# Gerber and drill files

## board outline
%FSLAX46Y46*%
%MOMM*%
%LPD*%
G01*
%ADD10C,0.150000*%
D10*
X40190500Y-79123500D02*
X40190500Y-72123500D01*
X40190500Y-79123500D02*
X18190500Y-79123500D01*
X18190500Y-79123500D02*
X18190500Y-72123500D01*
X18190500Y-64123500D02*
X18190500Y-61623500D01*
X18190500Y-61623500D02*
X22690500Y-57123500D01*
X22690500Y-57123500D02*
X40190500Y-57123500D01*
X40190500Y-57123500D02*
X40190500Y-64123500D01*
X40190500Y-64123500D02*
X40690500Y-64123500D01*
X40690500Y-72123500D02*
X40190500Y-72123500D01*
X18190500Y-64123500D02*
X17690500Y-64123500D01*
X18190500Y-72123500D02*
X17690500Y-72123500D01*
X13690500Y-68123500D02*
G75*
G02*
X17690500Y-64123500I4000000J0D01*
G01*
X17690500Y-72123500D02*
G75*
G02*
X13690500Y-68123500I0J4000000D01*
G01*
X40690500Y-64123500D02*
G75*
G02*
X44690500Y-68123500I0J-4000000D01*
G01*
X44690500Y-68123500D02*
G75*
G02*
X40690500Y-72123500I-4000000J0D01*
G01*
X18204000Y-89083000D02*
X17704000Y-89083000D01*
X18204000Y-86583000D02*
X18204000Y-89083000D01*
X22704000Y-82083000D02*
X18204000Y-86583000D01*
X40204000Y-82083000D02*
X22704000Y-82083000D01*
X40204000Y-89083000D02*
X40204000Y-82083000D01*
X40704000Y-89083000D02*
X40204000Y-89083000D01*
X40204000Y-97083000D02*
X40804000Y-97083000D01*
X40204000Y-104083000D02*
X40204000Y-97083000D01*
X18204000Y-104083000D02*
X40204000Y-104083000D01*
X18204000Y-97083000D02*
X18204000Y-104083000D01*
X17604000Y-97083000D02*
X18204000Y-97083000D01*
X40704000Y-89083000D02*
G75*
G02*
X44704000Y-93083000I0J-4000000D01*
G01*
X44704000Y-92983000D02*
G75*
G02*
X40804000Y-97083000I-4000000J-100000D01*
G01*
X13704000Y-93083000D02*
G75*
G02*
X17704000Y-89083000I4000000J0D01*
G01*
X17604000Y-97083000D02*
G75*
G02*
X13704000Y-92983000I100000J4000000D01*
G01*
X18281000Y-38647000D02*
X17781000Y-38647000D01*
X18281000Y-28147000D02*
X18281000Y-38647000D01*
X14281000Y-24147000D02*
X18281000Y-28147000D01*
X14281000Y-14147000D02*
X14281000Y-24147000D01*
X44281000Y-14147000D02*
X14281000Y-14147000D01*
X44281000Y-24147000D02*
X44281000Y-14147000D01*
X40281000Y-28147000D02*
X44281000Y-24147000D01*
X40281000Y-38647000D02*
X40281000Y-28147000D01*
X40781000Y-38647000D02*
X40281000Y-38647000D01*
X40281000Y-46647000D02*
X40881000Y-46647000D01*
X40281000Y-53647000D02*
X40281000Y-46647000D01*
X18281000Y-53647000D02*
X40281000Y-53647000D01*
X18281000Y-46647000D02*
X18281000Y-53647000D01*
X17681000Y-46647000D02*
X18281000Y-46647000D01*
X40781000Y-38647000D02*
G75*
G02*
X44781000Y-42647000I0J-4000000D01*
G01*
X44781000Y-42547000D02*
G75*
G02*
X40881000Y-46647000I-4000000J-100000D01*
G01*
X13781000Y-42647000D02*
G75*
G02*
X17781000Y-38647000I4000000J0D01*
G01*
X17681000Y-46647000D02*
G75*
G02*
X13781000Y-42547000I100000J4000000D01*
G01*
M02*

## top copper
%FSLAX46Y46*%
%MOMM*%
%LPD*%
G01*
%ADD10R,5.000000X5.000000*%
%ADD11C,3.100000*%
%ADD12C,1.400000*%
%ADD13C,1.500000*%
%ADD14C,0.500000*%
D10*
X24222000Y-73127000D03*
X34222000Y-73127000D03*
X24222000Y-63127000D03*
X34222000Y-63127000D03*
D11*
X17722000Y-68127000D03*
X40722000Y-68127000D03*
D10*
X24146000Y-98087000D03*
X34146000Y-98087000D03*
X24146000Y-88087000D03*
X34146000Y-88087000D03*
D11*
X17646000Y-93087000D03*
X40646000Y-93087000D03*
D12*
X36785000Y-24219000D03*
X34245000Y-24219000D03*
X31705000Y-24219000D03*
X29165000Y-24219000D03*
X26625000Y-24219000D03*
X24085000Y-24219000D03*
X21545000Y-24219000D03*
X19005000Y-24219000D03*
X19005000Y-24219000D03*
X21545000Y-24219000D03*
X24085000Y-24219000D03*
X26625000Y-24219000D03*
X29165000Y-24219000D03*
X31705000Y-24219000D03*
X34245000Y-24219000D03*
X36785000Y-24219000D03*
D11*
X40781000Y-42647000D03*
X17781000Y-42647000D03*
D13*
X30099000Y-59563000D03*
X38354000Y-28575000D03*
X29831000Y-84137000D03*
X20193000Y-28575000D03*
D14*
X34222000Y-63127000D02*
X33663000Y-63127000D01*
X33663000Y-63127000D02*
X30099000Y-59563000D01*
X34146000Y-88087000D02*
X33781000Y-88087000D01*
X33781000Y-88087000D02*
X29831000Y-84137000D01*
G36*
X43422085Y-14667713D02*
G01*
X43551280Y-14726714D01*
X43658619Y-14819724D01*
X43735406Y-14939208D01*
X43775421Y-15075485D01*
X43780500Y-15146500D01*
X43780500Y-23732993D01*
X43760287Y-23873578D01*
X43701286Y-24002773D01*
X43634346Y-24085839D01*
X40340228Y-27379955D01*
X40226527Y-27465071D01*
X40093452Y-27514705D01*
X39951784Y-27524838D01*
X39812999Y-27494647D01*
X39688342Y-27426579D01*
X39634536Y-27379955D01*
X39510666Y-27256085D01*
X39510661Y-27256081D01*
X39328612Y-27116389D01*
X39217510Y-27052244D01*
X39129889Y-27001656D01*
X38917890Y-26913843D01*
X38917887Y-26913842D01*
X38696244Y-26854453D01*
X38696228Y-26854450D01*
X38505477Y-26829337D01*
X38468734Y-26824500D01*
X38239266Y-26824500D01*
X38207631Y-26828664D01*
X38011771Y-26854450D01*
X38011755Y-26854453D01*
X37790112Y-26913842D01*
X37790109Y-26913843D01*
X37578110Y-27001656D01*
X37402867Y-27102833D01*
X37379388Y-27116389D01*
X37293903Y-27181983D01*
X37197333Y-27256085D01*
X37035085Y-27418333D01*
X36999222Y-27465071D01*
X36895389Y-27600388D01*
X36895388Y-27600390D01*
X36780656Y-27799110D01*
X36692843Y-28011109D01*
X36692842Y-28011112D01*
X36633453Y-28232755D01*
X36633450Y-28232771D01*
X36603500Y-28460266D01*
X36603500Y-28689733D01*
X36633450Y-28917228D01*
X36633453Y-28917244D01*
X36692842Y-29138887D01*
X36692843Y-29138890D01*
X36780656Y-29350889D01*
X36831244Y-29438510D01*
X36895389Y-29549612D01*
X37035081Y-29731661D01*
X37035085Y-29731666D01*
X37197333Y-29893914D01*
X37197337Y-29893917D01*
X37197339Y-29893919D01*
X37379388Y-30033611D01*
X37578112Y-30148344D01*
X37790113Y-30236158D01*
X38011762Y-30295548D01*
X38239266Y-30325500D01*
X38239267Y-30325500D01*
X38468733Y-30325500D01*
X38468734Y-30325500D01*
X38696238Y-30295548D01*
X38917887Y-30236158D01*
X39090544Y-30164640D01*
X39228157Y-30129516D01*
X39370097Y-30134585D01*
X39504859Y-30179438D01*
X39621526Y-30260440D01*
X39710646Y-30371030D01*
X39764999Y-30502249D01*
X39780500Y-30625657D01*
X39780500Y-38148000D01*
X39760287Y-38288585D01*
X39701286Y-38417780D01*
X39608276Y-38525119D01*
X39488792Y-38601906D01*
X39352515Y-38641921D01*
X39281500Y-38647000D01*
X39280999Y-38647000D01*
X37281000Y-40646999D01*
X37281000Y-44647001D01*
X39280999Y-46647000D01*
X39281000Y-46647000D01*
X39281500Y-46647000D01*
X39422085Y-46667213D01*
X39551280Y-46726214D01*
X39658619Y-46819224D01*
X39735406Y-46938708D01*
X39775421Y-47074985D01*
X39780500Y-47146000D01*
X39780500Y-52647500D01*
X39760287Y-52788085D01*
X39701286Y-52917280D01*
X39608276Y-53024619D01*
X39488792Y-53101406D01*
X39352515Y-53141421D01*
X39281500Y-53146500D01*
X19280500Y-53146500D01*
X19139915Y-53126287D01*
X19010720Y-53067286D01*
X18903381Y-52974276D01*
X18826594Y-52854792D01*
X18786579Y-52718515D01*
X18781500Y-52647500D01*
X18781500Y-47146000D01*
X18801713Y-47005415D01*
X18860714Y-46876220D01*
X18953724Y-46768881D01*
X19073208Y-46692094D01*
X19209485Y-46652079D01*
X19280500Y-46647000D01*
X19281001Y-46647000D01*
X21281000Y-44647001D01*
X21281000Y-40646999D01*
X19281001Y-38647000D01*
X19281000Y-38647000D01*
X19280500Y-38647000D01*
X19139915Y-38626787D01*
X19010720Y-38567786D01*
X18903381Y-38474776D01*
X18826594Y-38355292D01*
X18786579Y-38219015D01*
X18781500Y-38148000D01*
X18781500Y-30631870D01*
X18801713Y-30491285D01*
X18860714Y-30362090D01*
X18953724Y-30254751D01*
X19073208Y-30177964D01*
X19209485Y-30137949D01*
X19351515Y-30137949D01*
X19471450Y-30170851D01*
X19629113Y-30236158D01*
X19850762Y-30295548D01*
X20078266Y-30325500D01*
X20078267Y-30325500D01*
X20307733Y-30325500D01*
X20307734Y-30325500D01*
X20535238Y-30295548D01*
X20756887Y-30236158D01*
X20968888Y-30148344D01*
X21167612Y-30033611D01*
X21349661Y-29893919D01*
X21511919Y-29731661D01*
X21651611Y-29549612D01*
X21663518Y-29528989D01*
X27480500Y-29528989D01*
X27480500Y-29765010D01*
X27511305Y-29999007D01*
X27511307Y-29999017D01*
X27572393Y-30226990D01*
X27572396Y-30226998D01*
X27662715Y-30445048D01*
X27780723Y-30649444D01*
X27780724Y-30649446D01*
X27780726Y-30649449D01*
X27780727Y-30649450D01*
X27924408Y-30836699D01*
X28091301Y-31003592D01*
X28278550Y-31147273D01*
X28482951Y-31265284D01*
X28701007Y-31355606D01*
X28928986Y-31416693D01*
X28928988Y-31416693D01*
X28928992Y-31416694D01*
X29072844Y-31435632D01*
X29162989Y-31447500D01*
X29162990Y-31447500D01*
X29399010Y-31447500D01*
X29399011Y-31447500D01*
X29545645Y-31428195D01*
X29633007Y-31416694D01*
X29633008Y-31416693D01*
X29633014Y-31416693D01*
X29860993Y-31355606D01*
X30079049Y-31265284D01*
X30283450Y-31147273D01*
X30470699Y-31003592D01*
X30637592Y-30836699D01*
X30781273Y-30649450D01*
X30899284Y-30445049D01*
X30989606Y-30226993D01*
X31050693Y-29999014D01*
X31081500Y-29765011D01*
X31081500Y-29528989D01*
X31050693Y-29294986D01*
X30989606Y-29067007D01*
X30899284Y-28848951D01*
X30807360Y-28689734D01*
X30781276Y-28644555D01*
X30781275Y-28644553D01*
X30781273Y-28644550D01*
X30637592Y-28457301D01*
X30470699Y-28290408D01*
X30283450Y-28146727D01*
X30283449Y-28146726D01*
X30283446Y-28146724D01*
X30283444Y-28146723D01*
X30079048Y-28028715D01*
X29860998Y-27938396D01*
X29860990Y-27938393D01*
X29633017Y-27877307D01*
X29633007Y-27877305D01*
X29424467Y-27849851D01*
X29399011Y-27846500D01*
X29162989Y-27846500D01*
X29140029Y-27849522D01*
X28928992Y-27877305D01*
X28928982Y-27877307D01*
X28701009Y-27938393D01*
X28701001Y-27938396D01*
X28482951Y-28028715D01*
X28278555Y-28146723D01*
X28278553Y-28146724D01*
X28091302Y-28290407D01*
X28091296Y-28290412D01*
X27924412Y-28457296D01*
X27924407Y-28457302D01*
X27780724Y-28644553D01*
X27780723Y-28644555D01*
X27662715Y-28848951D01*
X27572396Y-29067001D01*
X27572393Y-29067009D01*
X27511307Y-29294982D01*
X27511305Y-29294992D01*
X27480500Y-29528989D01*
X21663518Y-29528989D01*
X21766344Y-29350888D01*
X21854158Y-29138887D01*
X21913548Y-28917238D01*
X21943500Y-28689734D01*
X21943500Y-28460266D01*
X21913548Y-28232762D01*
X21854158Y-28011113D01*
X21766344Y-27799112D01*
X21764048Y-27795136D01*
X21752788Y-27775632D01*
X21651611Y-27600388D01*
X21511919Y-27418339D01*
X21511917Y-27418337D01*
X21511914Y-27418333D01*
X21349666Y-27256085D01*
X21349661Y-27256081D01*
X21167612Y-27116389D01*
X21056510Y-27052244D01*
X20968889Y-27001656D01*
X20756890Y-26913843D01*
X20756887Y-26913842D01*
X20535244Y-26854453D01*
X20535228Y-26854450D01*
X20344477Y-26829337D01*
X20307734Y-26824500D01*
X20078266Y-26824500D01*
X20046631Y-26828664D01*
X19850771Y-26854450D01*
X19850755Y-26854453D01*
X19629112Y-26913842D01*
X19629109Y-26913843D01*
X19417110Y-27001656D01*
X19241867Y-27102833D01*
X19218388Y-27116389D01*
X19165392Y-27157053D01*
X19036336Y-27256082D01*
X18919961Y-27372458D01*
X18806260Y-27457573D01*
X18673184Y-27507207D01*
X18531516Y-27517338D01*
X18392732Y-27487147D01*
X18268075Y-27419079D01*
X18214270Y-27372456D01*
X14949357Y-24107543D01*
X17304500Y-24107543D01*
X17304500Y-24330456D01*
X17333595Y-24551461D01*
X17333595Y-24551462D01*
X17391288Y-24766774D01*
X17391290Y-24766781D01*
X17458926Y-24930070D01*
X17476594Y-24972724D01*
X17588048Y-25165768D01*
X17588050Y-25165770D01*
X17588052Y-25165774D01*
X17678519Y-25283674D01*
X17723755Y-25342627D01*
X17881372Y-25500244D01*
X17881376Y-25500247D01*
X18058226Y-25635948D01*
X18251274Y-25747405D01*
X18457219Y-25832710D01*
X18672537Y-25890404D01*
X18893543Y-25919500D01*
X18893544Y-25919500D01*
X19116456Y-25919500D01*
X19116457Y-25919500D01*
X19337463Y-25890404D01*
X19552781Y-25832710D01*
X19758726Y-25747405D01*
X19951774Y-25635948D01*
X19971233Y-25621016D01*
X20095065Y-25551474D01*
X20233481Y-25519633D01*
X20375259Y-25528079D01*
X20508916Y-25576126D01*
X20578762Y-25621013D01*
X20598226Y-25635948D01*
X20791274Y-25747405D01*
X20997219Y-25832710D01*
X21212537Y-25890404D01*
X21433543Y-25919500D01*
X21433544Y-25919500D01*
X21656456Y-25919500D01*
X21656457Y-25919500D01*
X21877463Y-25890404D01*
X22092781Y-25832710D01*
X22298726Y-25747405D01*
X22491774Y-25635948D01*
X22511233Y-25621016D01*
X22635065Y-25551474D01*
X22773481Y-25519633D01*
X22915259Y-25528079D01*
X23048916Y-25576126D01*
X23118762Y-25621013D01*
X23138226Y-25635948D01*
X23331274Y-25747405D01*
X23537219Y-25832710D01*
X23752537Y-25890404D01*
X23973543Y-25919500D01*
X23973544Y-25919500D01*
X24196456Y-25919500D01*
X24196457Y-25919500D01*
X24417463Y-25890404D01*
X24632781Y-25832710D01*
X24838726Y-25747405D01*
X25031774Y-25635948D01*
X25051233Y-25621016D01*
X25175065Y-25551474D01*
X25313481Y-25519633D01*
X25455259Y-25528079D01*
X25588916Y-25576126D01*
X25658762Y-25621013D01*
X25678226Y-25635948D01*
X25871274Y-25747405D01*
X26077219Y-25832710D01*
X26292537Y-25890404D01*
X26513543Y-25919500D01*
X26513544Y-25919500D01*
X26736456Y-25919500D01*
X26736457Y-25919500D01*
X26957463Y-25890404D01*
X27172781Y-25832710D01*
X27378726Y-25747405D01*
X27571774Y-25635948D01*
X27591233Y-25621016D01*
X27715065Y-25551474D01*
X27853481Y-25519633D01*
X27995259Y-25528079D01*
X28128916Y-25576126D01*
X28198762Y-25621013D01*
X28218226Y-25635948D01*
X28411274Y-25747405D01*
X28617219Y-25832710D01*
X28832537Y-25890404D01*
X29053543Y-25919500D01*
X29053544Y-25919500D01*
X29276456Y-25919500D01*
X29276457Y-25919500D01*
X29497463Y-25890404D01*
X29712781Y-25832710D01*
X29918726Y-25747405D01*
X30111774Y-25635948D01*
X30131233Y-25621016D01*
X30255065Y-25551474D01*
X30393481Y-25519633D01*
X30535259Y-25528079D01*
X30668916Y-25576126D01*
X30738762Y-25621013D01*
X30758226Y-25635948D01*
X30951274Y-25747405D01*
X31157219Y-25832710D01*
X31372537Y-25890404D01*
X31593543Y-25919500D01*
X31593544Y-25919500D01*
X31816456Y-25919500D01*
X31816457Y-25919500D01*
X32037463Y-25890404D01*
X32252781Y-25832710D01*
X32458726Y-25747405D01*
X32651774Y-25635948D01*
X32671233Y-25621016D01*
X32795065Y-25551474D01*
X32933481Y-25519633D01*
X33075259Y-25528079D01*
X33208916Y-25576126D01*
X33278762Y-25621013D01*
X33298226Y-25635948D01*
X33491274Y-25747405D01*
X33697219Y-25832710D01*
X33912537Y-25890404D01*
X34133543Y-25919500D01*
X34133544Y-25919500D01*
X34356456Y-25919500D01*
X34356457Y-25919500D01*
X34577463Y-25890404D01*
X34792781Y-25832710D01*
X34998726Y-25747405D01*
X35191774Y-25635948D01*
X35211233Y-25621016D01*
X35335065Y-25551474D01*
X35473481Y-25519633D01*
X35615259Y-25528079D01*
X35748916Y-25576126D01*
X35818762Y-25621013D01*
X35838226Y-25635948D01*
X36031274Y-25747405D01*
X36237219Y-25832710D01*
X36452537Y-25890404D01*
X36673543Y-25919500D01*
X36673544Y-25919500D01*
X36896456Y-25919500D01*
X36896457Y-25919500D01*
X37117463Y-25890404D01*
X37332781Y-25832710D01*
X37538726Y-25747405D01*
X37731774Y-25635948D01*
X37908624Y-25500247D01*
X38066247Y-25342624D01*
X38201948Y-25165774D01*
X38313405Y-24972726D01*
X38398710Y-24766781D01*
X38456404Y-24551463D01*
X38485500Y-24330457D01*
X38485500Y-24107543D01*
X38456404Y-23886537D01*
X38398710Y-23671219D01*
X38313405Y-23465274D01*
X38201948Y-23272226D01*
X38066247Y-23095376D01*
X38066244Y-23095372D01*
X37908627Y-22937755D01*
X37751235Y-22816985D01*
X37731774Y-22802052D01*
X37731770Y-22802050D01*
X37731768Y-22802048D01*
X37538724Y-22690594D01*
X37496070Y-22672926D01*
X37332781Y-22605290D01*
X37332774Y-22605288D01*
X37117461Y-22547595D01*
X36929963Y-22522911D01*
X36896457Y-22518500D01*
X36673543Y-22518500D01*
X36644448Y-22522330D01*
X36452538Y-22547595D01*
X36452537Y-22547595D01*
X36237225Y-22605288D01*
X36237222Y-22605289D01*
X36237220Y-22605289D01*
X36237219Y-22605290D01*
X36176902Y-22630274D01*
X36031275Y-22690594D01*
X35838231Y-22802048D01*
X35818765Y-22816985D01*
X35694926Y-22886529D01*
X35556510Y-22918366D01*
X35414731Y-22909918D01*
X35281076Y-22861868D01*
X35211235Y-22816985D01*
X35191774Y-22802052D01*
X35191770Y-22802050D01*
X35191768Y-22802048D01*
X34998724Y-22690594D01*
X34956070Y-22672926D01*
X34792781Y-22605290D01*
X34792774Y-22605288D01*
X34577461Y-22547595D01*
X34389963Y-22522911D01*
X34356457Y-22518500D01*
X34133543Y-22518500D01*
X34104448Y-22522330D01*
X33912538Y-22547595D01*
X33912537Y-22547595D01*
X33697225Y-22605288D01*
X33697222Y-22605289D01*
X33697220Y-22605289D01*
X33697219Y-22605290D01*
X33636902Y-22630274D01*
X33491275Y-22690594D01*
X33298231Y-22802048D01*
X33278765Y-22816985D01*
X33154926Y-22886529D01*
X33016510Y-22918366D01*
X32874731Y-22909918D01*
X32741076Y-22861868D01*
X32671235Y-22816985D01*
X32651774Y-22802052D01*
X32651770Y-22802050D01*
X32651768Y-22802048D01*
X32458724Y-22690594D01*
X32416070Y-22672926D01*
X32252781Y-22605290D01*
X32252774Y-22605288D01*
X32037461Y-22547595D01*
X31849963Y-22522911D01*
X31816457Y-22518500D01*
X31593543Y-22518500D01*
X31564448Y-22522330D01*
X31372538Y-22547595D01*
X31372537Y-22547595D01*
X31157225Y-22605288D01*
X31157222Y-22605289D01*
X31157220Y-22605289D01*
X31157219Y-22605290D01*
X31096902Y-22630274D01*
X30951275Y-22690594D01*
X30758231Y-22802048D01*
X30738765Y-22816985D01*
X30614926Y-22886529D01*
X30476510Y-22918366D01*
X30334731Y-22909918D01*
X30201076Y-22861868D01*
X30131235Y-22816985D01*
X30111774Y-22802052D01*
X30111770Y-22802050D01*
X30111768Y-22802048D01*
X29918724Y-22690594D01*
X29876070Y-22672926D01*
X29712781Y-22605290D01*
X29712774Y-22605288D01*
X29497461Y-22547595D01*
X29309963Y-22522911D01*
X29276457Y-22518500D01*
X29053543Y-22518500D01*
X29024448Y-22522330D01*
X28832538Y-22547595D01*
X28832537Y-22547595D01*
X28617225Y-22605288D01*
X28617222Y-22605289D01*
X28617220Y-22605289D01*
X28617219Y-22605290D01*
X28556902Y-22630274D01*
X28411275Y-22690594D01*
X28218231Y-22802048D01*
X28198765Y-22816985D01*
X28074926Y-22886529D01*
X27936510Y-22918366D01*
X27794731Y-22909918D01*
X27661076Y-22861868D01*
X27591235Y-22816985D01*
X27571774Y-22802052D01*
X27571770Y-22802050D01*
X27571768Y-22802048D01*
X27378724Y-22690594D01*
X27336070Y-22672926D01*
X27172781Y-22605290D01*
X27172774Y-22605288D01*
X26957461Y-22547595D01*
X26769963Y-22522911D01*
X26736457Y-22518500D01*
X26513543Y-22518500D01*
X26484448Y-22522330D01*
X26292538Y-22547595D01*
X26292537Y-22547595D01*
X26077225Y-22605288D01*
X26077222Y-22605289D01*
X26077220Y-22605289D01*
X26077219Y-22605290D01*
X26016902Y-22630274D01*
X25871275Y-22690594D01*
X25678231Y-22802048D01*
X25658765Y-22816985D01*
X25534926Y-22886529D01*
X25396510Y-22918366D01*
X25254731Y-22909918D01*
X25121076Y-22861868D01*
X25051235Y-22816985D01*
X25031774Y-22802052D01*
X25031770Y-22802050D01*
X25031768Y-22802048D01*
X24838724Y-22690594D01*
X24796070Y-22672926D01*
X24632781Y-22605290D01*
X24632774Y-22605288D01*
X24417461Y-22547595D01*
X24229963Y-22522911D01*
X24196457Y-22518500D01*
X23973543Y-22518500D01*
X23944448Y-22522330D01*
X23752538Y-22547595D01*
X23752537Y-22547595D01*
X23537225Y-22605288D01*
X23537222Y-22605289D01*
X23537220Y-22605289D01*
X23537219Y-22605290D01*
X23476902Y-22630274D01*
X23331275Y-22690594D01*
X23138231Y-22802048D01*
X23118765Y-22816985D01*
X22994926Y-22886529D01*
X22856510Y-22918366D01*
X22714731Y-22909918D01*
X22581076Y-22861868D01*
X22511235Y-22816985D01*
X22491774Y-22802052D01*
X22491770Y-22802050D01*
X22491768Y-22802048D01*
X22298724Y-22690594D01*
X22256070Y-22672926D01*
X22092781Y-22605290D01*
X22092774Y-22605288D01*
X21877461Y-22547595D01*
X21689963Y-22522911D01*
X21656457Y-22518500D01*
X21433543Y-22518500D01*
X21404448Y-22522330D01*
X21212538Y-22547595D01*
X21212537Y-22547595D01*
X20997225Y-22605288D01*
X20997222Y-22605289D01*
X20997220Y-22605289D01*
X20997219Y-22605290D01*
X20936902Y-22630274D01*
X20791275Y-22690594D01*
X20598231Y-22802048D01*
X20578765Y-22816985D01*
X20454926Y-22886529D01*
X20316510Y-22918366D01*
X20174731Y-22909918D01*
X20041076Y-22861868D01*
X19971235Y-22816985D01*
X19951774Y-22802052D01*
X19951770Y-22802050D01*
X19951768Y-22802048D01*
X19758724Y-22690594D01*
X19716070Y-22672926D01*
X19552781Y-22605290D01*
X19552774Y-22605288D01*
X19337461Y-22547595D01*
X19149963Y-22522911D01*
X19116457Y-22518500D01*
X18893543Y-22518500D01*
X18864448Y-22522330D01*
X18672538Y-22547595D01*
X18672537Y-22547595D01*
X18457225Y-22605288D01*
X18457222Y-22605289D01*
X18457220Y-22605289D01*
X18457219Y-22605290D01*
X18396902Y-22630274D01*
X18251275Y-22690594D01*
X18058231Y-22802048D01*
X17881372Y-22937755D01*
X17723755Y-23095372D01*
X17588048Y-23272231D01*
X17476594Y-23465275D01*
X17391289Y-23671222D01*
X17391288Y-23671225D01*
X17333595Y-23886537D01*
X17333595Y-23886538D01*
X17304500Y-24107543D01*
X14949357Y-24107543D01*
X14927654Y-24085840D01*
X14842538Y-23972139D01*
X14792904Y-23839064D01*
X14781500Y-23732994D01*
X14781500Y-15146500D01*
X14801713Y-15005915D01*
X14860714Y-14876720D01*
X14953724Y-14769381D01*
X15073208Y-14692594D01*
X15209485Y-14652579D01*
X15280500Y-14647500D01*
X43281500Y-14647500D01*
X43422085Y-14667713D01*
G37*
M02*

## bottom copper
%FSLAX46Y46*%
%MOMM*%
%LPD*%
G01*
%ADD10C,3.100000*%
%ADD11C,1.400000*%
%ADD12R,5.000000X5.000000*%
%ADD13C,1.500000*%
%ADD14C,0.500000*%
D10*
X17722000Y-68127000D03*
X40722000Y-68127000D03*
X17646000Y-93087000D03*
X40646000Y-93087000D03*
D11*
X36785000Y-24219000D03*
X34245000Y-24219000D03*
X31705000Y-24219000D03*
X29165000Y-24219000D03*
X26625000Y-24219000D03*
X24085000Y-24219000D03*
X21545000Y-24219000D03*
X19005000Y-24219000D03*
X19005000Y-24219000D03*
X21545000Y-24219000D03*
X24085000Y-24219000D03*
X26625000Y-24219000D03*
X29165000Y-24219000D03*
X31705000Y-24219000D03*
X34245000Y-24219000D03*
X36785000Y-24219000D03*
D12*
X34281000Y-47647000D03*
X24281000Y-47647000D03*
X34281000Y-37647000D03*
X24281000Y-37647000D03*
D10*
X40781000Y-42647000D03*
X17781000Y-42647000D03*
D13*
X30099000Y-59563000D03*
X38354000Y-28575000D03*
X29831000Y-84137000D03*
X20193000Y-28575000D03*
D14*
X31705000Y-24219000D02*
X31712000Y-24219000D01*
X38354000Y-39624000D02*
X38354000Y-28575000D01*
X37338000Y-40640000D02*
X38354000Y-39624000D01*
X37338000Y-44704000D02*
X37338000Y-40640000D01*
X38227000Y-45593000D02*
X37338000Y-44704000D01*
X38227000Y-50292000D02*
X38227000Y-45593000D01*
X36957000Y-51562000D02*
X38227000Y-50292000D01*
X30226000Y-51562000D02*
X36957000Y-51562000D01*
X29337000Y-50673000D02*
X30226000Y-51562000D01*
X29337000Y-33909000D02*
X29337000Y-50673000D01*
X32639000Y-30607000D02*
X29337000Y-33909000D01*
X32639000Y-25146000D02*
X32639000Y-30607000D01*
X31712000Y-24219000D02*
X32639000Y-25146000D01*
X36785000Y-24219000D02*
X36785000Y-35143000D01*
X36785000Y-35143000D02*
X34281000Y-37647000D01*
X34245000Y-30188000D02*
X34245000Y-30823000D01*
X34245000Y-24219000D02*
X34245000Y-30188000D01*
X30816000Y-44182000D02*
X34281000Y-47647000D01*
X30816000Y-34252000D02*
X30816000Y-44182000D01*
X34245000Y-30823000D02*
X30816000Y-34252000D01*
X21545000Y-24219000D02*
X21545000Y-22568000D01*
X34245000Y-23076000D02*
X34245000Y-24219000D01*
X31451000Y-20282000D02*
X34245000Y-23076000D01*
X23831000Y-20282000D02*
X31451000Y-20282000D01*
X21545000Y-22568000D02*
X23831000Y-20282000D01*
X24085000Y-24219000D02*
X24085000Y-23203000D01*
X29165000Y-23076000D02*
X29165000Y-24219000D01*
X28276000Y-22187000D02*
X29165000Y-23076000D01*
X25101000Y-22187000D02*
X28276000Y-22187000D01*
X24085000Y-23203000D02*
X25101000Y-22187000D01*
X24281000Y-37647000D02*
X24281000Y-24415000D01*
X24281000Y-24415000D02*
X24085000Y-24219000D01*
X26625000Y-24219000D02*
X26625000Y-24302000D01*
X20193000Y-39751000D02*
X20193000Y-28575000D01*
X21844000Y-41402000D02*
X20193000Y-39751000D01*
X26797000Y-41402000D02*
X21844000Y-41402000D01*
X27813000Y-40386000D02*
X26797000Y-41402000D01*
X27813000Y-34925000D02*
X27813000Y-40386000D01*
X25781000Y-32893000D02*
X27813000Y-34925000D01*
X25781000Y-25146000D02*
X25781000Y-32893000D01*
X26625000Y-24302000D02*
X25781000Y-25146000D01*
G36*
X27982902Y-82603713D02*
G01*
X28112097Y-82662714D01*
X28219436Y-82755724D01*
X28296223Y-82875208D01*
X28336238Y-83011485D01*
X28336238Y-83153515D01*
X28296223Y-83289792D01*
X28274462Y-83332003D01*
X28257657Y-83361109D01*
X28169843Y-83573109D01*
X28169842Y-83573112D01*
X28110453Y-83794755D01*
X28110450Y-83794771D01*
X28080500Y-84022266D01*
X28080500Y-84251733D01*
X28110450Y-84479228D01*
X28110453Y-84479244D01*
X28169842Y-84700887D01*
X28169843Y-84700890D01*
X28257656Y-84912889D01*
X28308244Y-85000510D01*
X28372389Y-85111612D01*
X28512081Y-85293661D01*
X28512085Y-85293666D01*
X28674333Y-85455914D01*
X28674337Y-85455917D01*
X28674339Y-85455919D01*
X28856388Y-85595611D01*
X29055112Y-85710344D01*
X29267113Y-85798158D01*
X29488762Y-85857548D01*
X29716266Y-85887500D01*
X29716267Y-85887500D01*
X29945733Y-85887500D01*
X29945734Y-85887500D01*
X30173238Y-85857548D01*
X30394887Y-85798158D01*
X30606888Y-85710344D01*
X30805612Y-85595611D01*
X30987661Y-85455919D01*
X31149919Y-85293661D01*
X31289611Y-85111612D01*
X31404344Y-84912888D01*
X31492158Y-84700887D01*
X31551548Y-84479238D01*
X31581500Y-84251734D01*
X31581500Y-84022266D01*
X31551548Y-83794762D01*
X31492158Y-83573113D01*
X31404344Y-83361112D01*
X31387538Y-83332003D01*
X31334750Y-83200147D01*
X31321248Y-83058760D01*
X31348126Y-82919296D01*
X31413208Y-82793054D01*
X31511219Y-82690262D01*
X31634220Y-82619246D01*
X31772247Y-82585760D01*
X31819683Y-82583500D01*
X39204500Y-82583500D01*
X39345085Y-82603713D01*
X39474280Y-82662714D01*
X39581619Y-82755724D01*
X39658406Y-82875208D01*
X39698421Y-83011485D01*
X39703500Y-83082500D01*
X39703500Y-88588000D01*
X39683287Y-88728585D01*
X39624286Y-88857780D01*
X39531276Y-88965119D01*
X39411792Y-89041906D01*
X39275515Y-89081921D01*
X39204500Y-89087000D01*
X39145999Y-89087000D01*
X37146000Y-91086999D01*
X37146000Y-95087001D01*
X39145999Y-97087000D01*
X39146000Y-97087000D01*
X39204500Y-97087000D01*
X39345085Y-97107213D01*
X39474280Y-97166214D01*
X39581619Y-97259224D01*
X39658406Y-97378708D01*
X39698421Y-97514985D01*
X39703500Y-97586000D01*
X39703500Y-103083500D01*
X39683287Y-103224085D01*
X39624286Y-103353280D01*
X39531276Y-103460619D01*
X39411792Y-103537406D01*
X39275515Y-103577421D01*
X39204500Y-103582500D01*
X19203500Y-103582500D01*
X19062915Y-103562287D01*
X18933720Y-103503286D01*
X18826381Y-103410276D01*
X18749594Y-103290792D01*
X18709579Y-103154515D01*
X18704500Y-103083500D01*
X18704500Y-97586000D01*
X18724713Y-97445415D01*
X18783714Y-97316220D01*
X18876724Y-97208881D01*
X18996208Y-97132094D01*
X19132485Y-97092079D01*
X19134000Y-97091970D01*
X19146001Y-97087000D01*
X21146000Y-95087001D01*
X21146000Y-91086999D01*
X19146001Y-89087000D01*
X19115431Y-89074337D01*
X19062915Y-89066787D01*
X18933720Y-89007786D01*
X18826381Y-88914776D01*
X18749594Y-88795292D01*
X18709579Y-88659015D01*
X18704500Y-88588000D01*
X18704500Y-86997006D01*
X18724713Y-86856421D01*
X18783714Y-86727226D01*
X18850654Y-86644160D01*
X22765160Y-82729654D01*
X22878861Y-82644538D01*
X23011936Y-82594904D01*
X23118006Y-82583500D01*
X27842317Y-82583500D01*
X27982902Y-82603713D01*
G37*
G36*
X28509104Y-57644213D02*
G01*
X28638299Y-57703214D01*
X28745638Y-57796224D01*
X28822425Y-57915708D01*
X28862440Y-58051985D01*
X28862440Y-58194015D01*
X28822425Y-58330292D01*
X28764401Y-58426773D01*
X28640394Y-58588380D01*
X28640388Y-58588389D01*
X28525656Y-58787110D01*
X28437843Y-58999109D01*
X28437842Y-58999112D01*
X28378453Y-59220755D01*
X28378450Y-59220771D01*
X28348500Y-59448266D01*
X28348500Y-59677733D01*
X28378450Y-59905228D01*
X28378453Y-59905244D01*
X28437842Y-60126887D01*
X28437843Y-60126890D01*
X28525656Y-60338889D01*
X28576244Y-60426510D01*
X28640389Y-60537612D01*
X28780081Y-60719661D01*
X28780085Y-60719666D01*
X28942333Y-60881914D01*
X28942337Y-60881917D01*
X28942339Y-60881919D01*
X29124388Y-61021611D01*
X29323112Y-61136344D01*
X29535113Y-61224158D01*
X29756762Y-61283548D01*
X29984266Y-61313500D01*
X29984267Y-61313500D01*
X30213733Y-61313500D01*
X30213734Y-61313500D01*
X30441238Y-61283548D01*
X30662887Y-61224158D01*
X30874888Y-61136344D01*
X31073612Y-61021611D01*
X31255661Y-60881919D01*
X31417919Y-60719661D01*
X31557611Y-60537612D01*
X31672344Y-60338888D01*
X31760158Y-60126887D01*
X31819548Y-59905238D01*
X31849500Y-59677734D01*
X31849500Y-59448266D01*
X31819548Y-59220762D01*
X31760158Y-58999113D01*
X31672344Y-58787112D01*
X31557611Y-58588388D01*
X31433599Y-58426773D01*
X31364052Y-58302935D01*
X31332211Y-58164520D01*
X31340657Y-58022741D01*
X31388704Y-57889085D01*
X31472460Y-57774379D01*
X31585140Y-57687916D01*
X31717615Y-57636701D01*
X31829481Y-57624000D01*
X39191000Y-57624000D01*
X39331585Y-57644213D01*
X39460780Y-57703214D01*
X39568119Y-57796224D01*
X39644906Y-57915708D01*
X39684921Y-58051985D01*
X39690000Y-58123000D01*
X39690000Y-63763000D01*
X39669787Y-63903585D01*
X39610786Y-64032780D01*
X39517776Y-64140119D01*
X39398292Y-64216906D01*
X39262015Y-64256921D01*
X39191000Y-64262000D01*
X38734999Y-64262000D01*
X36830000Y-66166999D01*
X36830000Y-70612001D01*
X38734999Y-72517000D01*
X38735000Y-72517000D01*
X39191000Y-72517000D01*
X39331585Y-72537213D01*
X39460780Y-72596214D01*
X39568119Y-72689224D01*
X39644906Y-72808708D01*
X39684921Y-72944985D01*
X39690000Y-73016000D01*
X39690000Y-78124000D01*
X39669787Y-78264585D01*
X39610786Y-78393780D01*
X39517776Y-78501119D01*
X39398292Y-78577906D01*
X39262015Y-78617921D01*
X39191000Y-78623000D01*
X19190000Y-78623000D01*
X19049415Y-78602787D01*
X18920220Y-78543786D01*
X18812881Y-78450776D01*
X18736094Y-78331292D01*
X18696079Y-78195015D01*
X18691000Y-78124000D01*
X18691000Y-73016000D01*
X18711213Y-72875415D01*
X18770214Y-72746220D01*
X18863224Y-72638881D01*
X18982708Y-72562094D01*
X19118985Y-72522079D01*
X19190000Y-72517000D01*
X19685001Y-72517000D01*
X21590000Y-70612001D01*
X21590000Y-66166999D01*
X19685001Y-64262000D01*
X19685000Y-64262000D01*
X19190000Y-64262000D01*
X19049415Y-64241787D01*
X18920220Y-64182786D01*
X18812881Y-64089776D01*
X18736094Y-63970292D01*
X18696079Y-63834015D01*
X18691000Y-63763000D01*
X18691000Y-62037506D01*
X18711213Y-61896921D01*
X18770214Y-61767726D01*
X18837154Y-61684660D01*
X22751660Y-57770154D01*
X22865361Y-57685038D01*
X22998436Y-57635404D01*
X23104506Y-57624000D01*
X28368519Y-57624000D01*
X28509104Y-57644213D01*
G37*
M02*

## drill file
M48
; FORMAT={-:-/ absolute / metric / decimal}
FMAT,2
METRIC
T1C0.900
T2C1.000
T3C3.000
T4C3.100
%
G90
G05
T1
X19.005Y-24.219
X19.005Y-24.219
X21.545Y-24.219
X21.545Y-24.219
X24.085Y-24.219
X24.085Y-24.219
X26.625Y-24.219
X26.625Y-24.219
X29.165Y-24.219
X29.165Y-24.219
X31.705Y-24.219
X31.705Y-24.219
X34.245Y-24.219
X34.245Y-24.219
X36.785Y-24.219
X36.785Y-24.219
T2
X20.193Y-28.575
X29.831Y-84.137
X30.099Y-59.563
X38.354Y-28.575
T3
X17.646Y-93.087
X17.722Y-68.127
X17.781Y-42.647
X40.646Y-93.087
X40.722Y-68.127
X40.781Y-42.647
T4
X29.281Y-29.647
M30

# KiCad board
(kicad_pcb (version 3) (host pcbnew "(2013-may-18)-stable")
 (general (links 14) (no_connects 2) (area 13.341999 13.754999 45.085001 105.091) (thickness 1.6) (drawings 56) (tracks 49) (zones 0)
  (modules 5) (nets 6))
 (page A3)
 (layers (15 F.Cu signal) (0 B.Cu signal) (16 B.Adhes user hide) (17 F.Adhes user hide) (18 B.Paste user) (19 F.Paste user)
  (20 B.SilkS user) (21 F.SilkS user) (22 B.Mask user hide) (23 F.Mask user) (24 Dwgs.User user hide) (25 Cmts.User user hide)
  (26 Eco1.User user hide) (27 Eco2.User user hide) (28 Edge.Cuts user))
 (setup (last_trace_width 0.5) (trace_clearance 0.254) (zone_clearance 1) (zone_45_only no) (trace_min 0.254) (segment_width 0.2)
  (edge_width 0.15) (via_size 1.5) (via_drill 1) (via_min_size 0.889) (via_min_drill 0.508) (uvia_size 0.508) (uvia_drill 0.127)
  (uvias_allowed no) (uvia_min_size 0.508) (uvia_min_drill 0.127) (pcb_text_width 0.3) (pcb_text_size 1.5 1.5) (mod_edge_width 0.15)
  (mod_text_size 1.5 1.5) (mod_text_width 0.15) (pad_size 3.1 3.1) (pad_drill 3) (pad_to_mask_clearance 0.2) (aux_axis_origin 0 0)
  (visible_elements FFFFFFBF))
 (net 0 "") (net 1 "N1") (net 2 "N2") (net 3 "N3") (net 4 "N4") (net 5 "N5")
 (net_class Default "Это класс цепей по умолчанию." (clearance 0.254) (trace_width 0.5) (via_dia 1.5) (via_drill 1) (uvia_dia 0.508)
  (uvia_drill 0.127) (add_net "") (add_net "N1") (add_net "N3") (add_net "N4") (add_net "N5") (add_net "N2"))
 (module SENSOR (layer F.Cu) (at 17.722 79.627)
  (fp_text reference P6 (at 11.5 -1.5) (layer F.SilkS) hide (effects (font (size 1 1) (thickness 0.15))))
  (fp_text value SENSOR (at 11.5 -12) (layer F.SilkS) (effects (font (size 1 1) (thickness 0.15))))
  (pad 2 smd rect (at 6.5 -6.5) (size 5 5) (layers F.Cu F.Mask) (solder_mask_margin 0.1))
  (pad 3 smd rect (at 16.5 -6.5) (size 5 5) (layers F.Cu F.Mask))
  (pad 1 smd rect (at 6.5 -16.5) (size 5 5) (layers F.Cu F.Mask))
  (pad 4 smd rect (at 16.5 -16.5) (size 5 5) (layers F.Cu F.Mask) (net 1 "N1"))
  (pad "" np_thru_hole circle (at 0 -11.5) (size 3.1 3.1) (drill 3) (layers *.Cu *.Mask F.SilkS))
  (pad "" np_thru_hole circle (at 23 -11.5) (size 3.1 3.1) (drill 3) (layers *.Cu *.Mask F.SilkS)))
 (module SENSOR (layer F.Cu) (at 17.646 104.587)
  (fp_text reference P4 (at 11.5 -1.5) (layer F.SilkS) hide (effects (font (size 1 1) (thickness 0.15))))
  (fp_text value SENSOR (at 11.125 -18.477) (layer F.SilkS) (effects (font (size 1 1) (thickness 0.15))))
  (pad 2 smd rect (at 6.5 -6.5) (size 5 5) (layers F.Cu F.Mask) (solder_mask_margin 0.1))
  (pad 3 smd rect (at 16.5 -6.5) (size 5 5) (layers F.Cu F.Mask))
  (pad 1 smd rect (at 6.5 -16.5) (size 5 5) (layers F.Cu F.Mask))
  (pad 4 smd rect (at 16.5 -16.5) (size 5 5) (layers F.Cu F.Mask) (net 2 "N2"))
  (pad "" np_thru_hole circle (at 0 -11.5) (size 3.1 3.1) (drill 3) (layers *.Cu *.Mask F.SilkS))
  (pad "" np_thru_hole circle (at 23 -11.5) (size 3.1 3.1) (drill 3) (layers *.Cu *.Mask F.SilkS)))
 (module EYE (layer F.Cu) (at 27.895 24.219 270)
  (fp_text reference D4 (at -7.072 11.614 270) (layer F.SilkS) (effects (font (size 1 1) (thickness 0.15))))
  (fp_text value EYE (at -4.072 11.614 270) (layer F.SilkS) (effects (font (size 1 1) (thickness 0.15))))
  (pad 1 thru_hole circle (at 0 -8.89 270) (size 1.4 1.4) (drill 0.9) (layers *.Cu *.Mask F.SilkS) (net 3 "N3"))
  (pad 2 thru_hole circle (at 0 -6.35 270) (size 1.4 1.4) (drill 0.9) (layers *.Cu *.Mask F.SilkS) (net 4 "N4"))
  (pad 3 thru_hole circle (at 0 -3.81 270) (size 1.4 1.4) (drill 0.9) (layers *.Cu *.Mask F.SilkS) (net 1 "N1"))
  (pad 4 thru_hole circle (at 0 -1.27 270) (size 1.4 1.4) (drill 0.9) (layers *.Cu *.Mask F.SilkS) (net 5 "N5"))
  (pad 5 thru_hole circle (at 0 1.27 270) (size 1.4 1.4) (drill 0.9) (layers *.Cu *.Mask F.SilkS) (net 2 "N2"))
  (pad 6 thru_hole circle (at 0 3.81 270) (size 1.4 1.4) (drill 0.9) (layers *.Cu *.Mask F.SilkS) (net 5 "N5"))
  (pad 7 thru_hole circle (at 0 6.35 270) (size 1.4 1.4) (drill 0.9) (layers *.Cu *.Mask F.SilkS) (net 4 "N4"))
  (pad 8 thru_hole circle (at 0 8.89 270) (size 1.4 1.4) (drill 0.9) (layers *.Cu *.Mask F.SilkS))
  (pad 8 thru_hole circle (at 0 8.89 270) (size 1.4 1.4) (drill 0.9) (layers *.Cu *.Mask F.SilkS))
  (pad 7 thru_hole circle (at 0 6.35 270) (size 1.4 1.4) (drill 0.9) (layers *.Cu *.Mask F.SilkS) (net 4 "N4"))
  (pad 6 thru_hole circle (at 0 3.81 270) (size 1.4 1.4) (drill 0.9) (layers *.Cu *.Mask F.SilkS) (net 5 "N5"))
  (pad 5 thru_hole circle (at 0 1.27 270) (size 1.4 1.4) (drill 0.9) (layers *.Cu *.Mask F.SilkS) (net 2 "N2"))
  (pad 4 thru_hole circle (at 0 -1.27 270) (size 1.4 1.4) (drill 0.9) (layers *.Cu *.Mask F.SilkS) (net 5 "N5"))
  (pad 3 thru_hole circle (at 0 -3.81 270) (size 1.4 1.4) (drill 0.9) (layers *.Cu *.Mask F.SilkS) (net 1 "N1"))
  (pad 2 thru_hole circle (at 0 -6.35 270) (size 1.4 1.4) (drill 0.9) (layers *.Cu *.Mask F.SilkS) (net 4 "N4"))
  (pad 1 thru_hole circle (at 0 -8.89 270) (size 1.4 1.4) (drill 0.9) (layers *.Cu *.Mask F.SilkS) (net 3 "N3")))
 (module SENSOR (layer B.Cu) (at 40.781 54.147 180)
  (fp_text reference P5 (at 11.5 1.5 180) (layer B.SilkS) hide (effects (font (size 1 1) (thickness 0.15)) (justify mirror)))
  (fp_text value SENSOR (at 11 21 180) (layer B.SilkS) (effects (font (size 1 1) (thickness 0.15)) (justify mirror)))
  (pad 2 smd rect (at 6.5 6.5 180) (size 5 5) (layers B.Cu B.Mask) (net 4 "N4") (solder_mask_margin 0.1))
  (pad 3 smd rect (at 16.5 6.5 180) (size 5 5) (layers B.Cu B.Mask))
  (pad 1 smd rect (at 6.5 16.5 180) (size 5 5) (layers B.Cu B.Mask) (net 3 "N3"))
  (pad 4 smd rect (at 16.5 16.5 180) (size 5 5) (layers B.Cu B.Mask) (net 5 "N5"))
  (pad "" np_thru_hole circle (at 0 11.5 180) (size 3.1 3.1) (drill 3) (layers *.Cu *.Mask B.SilkS))
  (pad "" np_thru_hole circle (at 23 11.5 180) (size 3.1 3.1) (drill 3) (layers *.Cu *.Mask B.SilkS)))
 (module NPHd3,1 (layer F.Cu) (at 29.281 29.647 90)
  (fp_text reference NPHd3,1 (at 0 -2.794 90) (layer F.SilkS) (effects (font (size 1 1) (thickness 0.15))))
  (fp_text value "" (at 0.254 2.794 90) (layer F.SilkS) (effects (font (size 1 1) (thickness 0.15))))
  (pad "" np_thru_hole circle (at 0 0 90) (size 3.1 3.1) (drill 3.1) (layers *.Cu *.Mask F.SilkS)))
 (gr_line (start 40.1905 79.1235) (end 40.1905 72.1235) (angle 90) (layer Edge.Cuts) (width 0.15))
 (gr_line (start 40.1905 79.1235) (end 18.1905 79.1235) (angle 90) (layer Edge.Cuts) (width 0.15))
 (gr_line (start 18.1905 79.1235) (end 18.1905 72.1235) (angle 90) (layer Edge.Cuts) (width 0.15))
 (gr_line (start 18.1905 64.1235) (end 18.1905 61.6235) (angle 90) (layer Edge.Cuts) (width 0.15))
 (gr_line (start 18.1905 61.6235) (end 22.6905 57.1235) (angle 90) (layer Edge.Cuts) (width 0.15))
 (gr_line (start 22.6905 57.1235) (end 40.1905 57.1235) (angle 90) (layer Edge.Cuts) (width 0.15))
 (gr_line (start 40.1905 57.1235) (end 40.1905 64.1235) (angle 90) (layer Edge.Cuts) (width 0.15))
 (gr_line (start 40.1905 64.1235) (end 40.6905 64.1235) (angle 90) (layer Edge.Cuts) (width 0.15))
 (gr_line (start 40.6905 72.1235) (end 40.1905 72.1235) (angle 90) (layer Edge.Cuts) (width 0.15))
 (gr_line (start 18.1905 64.1235) (end 17.6905 64.1235) (angle 90) (layer Edge.Cuts) (width 0.15))
 (gr_line (start 18.1905 72.1235) (end 17.6905 72.1235) (angle 90) (layer Edge.Cuts) (width 0.15))
 (gr_arc (start 17.6905 68.1235) (end 17.6905 64.1235) (angle -90) (layer Edge.Cuts) (width 0.15))
 (gr_arc (start 17.6905 68.1235) (end 13.6905 68.1235) (angle -90) (layer Edge.Cuts) (width 0.15))
 (gr_arc (start 40.6905 68.1235) (end 44.6905 68.1235) (angle -90) (layer Edge.Cuts) (width 0.15))
 (gr_arc (start 40.6905 68.1235) (end 40.6905 72.1235) (angle -90) (layer Edge.Cuts) (width 0.15))
 (gr_line (start 18.204 89.083) (end 17.704 89.083) (angle 90) (layer Edge.Cuts) (width 0.15))
 (gr_line (start 18.204 86.583) (end 18.204 89.083) (angle 90) (layer Edge.Cuts) (width 0.15))
 (gr_line (start 22.704 82.083) (end 18.204 86.583) (angle 90) (layer Edge.Cuts) (width 0.15))
 (gr_line (start 40.204 82.083) (end 22.704 82.083) (angle 90) (layer Edge.Cuts) (width 0.15))
 (gr_line (start 40.204 89.083) (end 40.204 82.083) (angle 90) (layer Edge.Cuts) (width 0.15))
 (gr_line (start 40.704 89.083) (end 40.204 89.083) (angle 90) (layer Edge.Cuts) (width 0.15))
 (gr_line (start 40.204 97.083) (end 40.804 97.083) (angle 90) (layer Edge.Cuts) (width 0.15))
 (gr_line (start 40.204 104.083) (end 40.204 97.083) (angle 90) (layer Edge.Cuts) (width 0.15))
 (gr_line (start 18.204 104.083) (end 40.204 104.083) (angle 90) (layer Edge.Cuts) (width 0.15))
 (gr_line (start 18.204 97.083) (end 18.204 104.083) (angle 90) (layer Edge.Cuts) (width 0.15))
 (gr_line (start 17.604 97.083) (end 18.204 97.083) (angle 90) (layer Edge.Cuts) (width 0.15))
 (gr_arc (start 40.704 93.083) (end 40.704 89.083) (angle 90) (layer Edge.Cuts) (width 0.15))
 (gr_arc (start 40.704 93.083) (end 44.704 92.983) (angle 90) (layer Edge.Cuts) (width 0.15))
 (gr_arc (start 17.704 93.083) (end 13.704 93.083) (angle 90) (layer Edge.Cuts) (width 0.15))
 (gr_arc (start 17.704 93.083) (end 17.604 97.083) (angle 90) (layer Edge.Cuts) (width 0.15))
 (gr_line (start 18.281 38.647) (end 17.781 38.647) (angle 90) (layer Edge.Cuts) (width 0.15))
 (gr_line (start 18.281 28.147) (end 18.281 38.647) (angle 90) (layer Edge.Cuts) (width 0.15))
 (gr_line (start 14.281 24.147) (end 18.281 28.147) (angle 90) (layer Edge.Cuts) (width 0.15))
 (gr_line (start 14.281 14.147) (end 14.281 24.147) (angle 90) (layer Edge.Cuts) (width 0.15))
 (gr_line (start 44.281 14.147) (end 14.281 14.147) (angle 90) (layer Edge.Cuts) (width 0.15))
 (gr_line (start 44.281 24.147) (end 44.281 14.147) (angle 90) (layer Edge.Cuts) (width 0.15))
 (gr_line (start 40.281 28.147) (end 44.281 24.147) (angle 90) (layer Edge.Cuts) (width 0.15))
 (gr_line (start 40.281 38.647) (end 40.281 28.147) (angle 90) (layer Edge.Cuts) (width 0.15))
 (gr_line (start 40.781 38.647) (end 40.281 38.647) (angle 90) (layer Edge.Cuts) (width 0.15))
 (gr_line (start 40.281 46.647) (end 40.881 46.647) (angle 90) (layer Edge.Cuts) (width 0.15))
 (gr_line (start 40.281 53.647) (end 40.281 46.647) (angle 90) (layer Edge.Cuts) (width 0.15))
 (gr_line (start 18.281 53.647) (end 40.281 53.647) (angle 90) (layer Edge.Cuts) (width 0.15))
 (gr_line (start 18.281 46.647) (end 18.281 53.647) (angle 90) (layer Edge.Cuts) (width 0.15))
 (gr_line (start 17.681 46.647) (end 18.281 46.647) (angle 90) (layer Edge.Cuts) (width 0.15))
 (gr_arc (start 40.781 42.647) (end 40.781 38.647) (angle 90) (layer Edge.Cuts) (width 0.15))
 (gr_arc (start 40.781 42.647) (end 44.781 42.547) (angle 90) (layer Edge.Cuts) (width 0.15))
 (gr_arc (start 17.781 42.647) (end 13.781 42.647) (angle 90) (layer Edge.Cuts) (width 0.15))
 (gr_arc (start 17.781 42.647) (end 17.681 46.647) (angle 90) (layer Edge.Cuts) (width 0.15))
 (segment (start 34.222 63.127) (end 33.663 63.127) (width 0.5) (layer F.Cu) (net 1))
 (via (at 30.099 59.563) (size 1.5) (layers F.Cu B.Cu) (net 1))
 (segment (start 33.663 63.127) (end 30.099 59.563) (width 0.5) (layer F.Cu) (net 1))
 (segment (start 31.705 24.219) (end 31.712 24.219) (width 0.5) (layer B.Cu) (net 1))
 (via (at 38.354 28.575) (size 1.5) (layers F.Cu B.Cu) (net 1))
 (segment (start 38.354 39.624) (end 38.354 28.575) (width 0.5) (layer B.Cu) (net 1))
 (segment (start 37.338 40.64) (end 38.354 39.624) (width 0.5) (layer B.Cu) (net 1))
 (segment (start 37.338 44.704) (end 37.338 40.64) (width 0.5) (layer B.Cu) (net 1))
 (segment (start 38.227 45.593) (end 37.338 44.704) (width 0.5) (layer B.Cu) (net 1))
 (segment (start 38.227 50.292) (end 38.227 45.593) (width 0.5) (layer B.Cu) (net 1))
 (segment (start 36.957 51.562) (end 38.227 50.292) (width 0.5) (layer B.Cu) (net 1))
 (segment (start 30.226 51.562) (end 36.957 51.562) (width 0.5) (layer B.Cu) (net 1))
 (segment (start 29.337 50.673) (end 30.226 51.562) (width 0.5) (layer B.Cu) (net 1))
 (segment (start 29.337 33.909) (end 29.337 50.673) (width 0.5) (layer B.Cu) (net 1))
 (segment (start 32.639 30.607) (end 29.337 33.909) (width 0.5) (layer B.Cu) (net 1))
 (segment (start 32.639 25.146) (end 32.639 30.607) (width 0.5) (layer B.Cu) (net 1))
 (segment (start 31.712 24.219) (end 32.639 25.146) (width 0.5) (layer B.Cu) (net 1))
 (segment (start 36.785 24.219) (end 36.785 35.143) (width 0.5) (layer B.Cu) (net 3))
 (segment (start 36.785 35.143) (end 34.281 37.647) (width 0.5) (layer B.Cu) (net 3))
 (segment (start 34.245 30.188) (end 34.245 30.823) (width 0.5) (layer B.Cu) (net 4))
 (segment (start 34.245 24.219) (end 34.245 30.188) (width 0.5) (layer B.Cu) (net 4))
 (segment (start 30.816 44.182) (end 34.281 47.647) (width 0.5) (layer B.Cu) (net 4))
 (segment (start 30.816 34.252) (end 30.816 44.182) (width 0.5) (layer B.Cu) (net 4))
 (segment (start 34.245 30.823) (end 30.816 34.252) (width 0.5) (layer B.Cu) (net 4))
 (segment (start 21.545 24.219) (end 21.545 22.568) (width 0.5) (layer B.Cu) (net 4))
 (segment (start 34.245 23.076) (end 34.245 24.219) (width 0.5) (layer B.Cu) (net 4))
 (segment (start 31.451 20.282) (end 34.245 23.076) (width 0.5) (layer B.Cu) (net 4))
 (segment (start 23.831 20.282) (end 31.451 20.282) (width 0.5) (layer B.Cu) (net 4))
 (segment (start 21.545 22.568) (end 23.831 20.282) (width 0.5) (layer B.Cu) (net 4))
 (segment (start 24.085 24.219) (end 24.085 23.203) (width 0.5) (layer B.Cu) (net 5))
 (segment (start 29.165 23.076) (end 29.165 24.219) (width 0.5) (layer B.Cu) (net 5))
 (segment (start 28.276 22.187) (end 29.165 23.076) (width 0.5) (layer B.Cu) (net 5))
 (segment (start 25.101 22.187) (end 28.276 22.187) (width 0.5) (layer B.Cu) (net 5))
 (segment (start 24.085 23.203) (end 25.101 22.187) (width 0.5) (layer B.Cu) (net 5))
 (segment (start 24.281 37.647) (end 24.281 24.415) (width 0.5) (layer B.Cu) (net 5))
 (segment (start 24.281 24.415) (end 24.085 24.219) (width 0.5) (layer B.Cu) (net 5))
 (segment (start 34.146 88.087) (end 33.781 88.087) (width 0.5) (layer F.Cu) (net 2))
 (via (at 29.831 84.137) (size 1.5) (layers F.Cu B.Cu) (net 2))
 (segment (start 33.781 88.087) (end 29.831 84.137) (width 0.5) (layer F.Cu) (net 2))
 (segment (start 26.625 24.219) (end 26.625 24.302) (width 0.5) (layer B.Cu) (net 2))
 (via (at 20.193 28.575) (size 1.5) (layers F.Cu B.Cu) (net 2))
 (segment (start 20.193 39.751) (end 20.193 28.575) (width 0.5) (layer B.Cu) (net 2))
 (segment (start 21.844 41.402) (end 20.193 39.751) (width 0.5) (layer B.Cu) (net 2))
 (segment (start 26.797 41.402) (end 21.844 41.402) (width 0.5) (layer B.Cu) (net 2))
 (segment (start 27.813 40.386) (end 26.797 41.402) (width 0.5) (layer B.Cu) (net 2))
 (segment (start 27.813 34.925) (end 27.813 40.386) (width 0.5) (layer B.Cu) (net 2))
 (segment (start 25.781 32.893) (end 27.813 34.925) (width 0.5) (layer B.Cu) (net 2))
 (segment (start 25.781 25.146) (end 25.781 32.893) (width 0.5) (layer B.Cu) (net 2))
 (segment (start 26.625 24.302) (end 25.781 25.146) (width 0.5) (layer B.Cu) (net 2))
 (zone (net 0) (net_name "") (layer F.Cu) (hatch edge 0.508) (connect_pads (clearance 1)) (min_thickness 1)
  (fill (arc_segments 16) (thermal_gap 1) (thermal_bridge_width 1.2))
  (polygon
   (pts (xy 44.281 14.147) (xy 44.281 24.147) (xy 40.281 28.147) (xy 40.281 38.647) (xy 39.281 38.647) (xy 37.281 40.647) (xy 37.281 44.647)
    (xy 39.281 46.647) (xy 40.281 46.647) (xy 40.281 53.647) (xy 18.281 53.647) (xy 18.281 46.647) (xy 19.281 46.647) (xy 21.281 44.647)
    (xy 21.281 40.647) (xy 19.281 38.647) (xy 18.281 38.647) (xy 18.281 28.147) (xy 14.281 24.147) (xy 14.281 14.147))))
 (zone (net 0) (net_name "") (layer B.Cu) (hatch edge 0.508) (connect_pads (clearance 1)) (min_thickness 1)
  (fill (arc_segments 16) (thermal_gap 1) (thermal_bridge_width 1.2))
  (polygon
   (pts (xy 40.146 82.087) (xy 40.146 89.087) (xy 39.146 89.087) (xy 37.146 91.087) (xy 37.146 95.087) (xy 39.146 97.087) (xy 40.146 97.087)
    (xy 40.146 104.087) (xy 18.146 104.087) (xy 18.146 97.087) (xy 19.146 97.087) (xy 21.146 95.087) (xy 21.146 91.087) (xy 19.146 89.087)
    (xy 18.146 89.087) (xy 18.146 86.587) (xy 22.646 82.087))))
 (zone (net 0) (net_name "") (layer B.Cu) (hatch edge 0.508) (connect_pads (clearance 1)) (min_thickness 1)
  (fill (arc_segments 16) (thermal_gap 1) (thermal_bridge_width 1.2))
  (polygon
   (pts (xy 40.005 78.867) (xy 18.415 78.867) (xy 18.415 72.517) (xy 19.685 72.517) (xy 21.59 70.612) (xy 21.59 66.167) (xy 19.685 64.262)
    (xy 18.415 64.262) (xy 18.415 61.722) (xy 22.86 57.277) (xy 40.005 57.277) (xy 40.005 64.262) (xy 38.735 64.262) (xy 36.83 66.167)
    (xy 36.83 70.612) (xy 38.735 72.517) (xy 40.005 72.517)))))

